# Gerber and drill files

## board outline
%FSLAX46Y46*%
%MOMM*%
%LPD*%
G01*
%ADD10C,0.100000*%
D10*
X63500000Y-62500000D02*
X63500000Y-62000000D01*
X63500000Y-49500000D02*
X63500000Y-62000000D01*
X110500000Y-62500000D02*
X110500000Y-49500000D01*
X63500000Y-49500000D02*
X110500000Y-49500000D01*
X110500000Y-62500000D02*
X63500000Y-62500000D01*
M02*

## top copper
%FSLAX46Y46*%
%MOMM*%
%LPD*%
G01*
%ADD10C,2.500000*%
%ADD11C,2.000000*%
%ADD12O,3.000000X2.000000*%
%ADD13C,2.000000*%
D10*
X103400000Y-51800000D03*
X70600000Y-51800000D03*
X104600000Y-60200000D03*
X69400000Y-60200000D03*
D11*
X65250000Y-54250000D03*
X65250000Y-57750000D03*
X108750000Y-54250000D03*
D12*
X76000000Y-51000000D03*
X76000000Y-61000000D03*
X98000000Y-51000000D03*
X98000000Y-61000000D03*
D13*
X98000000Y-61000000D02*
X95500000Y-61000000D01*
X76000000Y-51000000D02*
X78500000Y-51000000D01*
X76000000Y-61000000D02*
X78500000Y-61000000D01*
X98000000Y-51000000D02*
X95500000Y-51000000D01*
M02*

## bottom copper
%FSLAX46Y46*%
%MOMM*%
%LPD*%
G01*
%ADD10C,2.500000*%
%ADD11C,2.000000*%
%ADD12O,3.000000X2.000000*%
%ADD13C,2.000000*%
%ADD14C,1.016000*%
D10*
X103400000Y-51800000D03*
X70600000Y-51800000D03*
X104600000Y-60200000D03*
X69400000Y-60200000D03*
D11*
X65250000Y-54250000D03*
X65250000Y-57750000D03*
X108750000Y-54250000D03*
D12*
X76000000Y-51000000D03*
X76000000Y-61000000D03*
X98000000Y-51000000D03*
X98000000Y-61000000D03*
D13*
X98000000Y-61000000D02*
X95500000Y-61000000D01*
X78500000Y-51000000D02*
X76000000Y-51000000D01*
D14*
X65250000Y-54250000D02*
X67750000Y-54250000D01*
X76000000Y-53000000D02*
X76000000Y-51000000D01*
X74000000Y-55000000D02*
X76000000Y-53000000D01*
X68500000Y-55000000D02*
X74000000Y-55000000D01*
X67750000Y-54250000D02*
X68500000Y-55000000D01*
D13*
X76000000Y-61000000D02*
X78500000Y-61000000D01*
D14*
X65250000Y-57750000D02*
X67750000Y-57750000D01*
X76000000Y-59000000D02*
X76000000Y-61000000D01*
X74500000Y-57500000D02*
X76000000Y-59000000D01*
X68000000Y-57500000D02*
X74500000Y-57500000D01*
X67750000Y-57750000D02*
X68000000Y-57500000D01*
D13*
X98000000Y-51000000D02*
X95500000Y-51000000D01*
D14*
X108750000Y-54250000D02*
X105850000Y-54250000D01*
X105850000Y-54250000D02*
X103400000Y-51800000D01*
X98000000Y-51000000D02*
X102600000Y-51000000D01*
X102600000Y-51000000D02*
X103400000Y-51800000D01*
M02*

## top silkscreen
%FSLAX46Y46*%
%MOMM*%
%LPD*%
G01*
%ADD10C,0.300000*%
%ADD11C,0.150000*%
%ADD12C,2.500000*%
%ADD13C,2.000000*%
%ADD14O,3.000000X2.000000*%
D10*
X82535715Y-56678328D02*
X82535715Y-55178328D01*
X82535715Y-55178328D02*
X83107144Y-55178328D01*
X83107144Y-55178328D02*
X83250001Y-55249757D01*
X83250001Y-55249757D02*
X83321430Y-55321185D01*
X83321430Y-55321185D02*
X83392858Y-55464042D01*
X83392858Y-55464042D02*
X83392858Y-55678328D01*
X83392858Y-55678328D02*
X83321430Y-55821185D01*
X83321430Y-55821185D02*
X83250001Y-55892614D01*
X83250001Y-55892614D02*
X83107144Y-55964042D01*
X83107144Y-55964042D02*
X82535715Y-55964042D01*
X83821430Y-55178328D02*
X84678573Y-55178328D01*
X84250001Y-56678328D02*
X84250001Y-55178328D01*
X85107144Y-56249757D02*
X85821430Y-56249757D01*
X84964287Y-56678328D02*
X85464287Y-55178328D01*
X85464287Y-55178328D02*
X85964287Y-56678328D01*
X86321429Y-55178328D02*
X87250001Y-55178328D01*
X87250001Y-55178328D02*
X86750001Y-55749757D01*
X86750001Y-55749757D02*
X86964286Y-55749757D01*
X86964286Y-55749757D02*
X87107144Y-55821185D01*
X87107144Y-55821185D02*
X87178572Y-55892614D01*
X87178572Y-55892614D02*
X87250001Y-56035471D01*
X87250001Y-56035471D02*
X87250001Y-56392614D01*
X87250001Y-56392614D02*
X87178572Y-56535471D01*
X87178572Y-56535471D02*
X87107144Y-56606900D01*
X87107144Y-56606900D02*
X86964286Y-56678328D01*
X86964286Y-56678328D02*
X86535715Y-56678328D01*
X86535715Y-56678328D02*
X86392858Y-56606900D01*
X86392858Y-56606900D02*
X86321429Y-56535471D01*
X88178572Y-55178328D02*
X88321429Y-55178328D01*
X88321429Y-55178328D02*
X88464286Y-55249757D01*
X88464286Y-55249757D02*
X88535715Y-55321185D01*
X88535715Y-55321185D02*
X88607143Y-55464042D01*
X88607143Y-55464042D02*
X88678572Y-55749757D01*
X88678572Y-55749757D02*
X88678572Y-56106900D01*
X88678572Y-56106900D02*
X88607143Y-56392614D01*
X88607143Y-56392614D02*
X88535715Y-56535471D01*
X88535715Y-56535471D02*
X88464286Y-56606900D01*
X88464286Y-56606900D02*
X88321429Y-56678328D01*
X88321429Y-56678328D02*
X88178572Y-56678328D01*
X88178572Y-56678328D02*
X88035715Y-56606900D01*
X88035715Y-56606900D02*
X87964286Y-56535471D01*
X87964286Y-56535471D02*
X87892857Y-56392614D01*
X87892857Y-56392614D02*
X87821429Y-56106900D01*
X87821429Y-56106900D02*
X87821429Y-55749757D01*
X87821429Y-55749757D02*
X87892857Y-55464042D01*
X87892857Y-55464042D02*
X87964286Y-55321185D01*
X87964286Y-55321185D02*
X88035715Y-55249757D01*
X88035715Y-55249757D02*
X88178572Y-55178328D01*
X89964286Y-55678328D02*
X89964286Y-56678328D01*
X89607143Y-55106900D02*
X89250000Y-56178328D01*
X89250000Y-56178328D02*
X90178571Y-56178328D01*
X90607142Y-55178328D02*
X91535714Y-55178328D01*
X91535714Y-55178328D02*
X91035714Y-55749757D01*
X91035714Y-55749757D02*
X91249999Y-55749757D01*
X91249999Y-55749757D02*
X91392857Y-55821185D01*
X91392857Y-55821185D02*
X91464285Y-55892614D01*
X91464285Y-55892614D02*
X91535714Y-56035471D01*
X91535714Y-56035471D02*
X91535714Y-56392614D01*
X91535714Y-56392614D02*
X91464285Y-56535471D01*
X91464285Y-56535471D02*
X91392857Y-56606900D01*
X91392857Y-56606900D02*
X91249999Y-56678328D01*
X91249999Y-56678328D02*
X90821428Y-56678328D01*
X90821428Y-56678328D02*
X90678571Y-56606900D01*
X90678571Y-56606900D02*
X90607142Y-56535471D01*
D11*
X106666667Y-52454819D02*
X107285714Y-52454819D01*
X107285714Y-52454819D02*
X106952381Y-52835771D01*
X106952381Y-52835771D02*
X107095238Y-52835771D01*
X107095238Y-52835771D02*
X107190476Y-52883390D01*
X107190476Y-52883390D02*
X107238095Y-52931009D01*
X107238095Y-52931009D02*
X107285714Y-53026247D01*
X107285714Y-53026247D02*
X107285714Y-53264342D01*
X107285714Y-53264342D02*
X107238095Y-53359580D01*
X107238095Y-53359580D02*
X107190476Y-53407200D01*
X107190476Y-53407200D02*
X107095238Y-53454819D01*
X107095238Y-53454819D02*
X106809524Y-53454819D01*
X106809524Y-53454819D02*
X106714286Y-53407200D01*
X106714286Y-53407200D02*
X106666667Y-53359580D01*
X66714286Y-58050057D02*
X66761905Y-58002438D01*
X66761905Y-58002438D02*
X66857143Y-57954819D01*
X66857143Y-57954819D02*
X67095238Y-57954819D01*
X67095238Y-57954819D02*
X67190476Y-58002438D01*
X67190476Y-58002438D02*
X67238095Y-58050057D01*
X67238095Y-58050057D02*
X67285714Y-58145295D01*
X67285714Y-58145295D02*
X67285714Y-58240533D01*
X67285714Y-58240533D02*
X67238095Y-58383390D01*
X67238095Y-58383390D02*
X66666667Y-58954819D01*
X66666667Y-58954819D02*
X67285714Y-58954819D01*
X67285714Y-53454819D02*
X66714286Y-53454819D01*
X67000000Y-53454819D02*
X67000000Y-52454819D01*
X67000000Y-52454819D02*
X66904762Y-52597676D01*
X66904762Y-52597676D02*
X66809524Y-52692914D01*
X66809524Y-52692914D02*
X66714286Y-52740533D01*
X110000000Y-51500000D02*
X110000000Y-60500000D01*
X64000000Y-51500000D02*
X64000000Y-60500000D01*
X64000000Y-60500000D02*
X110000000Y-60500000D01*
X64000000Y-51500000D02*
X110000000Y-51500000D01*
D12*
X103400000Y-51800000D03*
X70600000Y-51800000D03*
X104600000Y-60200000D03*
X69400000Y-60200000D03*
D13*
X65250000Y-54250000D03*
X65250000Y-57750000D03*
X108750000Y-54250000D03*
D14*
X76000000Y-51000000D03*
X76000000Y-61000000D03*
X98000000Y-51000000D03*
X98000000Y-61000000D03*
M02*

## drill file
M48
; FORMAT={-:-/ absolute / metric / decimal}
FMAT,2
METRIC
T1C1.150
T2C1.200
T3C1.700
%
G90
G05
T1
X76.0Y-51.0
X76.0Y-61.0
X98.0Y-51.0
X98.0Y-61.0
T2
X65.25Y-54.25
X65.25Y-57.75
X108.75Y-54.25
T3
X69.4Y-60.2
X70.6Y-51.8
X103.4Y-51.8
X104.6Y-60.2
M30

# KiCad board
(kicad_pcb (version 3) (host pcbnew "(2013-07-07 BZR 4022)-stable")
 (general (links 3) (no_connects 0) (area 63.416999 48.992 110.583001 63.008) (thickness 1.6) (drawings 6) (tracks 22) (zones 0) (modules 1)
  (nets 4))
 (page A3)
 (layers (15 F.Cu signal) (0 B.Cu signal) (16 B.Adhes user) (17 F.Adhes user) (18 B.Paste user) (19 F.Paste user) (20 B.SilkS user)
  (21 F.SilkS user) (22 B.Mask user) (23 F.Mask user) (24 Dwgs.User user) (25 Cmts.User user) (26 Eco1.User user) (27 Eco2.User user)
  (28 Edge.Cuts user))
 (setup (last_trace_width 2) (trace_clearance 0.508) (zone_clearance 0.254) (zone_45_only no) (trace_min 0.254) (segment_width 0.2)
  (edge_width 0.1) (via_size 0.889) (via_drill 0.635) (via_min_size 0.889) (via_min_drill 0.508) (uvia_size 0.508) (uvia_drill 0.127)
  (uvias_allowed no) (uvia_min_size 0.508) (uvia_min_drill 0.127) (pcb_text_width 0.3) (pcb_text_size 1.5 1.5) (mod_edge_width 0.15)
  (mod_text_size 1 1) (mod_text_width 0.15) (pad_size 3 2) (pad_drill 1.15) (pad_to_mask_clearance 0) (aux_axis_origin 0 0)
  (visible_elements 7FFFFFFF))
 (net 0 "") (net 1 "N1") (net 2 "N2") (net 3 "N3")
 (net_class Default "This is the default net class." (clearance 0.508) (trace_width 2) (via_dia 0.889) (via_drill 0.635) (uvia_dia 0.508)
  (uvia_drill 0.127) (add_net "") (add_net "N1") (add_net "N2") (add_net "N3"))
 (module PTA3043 (layer F.Cu) (at 87 56)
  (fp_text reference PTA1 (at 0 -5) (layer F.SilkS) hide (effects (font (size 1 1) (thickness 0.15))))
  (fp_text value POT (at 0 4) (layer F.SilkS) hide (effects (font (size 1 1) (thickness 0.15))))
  (fp_line (start 23 -4.5) (end 23 4.5) (layer F.SilkS) (width 0.15))
  (fp_line (start -23 -4.5) (end -23 4.5) (layer F.SilkS) (width 0.15))
  (fp_line (start -23 4.5) (end 23 4.5) (layer F.SilkS) (width 0.15))
  (fp_line (start -23 -4.5) (end 23 -4.5) (layer F.SilkS) (width 0.15))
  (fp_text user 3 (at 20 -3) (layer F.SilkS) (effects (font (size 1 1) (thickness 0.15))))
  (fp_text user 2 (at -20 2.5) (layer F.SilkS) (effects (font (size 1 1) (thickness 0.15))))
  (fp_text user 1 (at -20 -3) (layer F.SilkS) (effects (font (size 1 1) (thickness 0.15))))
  (pad 7 thru_hole circle (at 16.4 -4.2) (size 2.5 2.5) (drill 1.7) (layers *.Cu *.Mask F.SilkS))
  (pad 6 thru_hole circle (at -16.4 -4.2) (size 2.5 2.5) (drill 1.7) (layers *.Cu *.Mask F.SilkS))
  (pad 5 thru_hole circle (at 17.6 4.2) (size 2.5 2.5) (drill 1.7) (layers *.Cu *.Mask F.SilkS))
  (pad 4 thru_hole circle (at -17.6 4.2) (size 2.5 2.5) (drill 1.7) (layers *.Cu *.Mask F.SilkS))
  (pad 1 thru_hole circle (at -21.75 -1.75) (size 2 2) (drill 1.2) (layers *.Cu *.Mask F.SilkS) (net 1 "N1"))
  (pad 2 thru_hole circle (at -21.75 1.75) (size 2 2) (drill 1.2) (layers *.Cu *.Mask F.SilkS) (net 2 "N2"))
  (pad 3 thru_hole circle (at 21.75 -1.75) (size 2 2) (drill 1.2) (layers *.Cu *.Mask F.SilkS) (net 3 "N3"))
  (pad 1 thru_hole oval (at -11 -5) (size 3 2) (drill 1.15) (layers *.Cu *.Mask F.SilkS) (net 1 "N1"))
  (pad 2 thru_hole oval (at -11 5) (size 3 2) (drill 1.15) (layers *.Cu *.Mask F.SilkS) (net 2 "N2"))
  (pad 3 thru_hole oval (at 11 -5) (size 3 2) (drill 1.15) (layers *.Cu *.Mask F.SilkS) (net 3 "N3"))
  (pad 8 thru_hole oval (at 11 5) (size 3 2) (drill 1.15) (layers *.Cu *.Mask F.SilkS)))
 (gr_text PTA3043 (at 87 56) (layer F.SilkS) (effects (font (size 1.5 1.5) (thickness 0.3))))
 (gr_line (start 63.5 62.5) (end 63.5 62) (angle 90) (layer Edge.Cuts) (width 0.1))
 (gr_line (start 63.5 49.5) (end 63.5 62) (angle 90) (layer Edge.Cuts) (width 0.1))
 (gr_line (start 110.5 62.5) (end 110.5 49.5) (angle 90) (layer Edge.Cuts) (width 0.1))
 (gr_line (start 63.5 49.5) (end 110.5 49.5) (angle 90) (layer Edge.Cuts) (width 0.1))
 (gr_line (start 110.5 62.5) (end 63.5 62.5) (angle 90) (layer Edge.Cuts) (width 0.1))
 (segment (start 98 61) (end 95.5 61) (width 2) (layer F.Cu) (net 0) (status 400000))
 (segment (start 98 61) (end 95.5 61) (width 2) (layer B.Cu) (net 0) (status 400000))
 (segment (start 76 51) (end 78.5 51) (width 2) (layer F.Cu) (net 1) (status 400000))
 (segment (start 78.5 51) (end 76 51) (width 2) (layer B.Cu) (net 1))
 (segment (start 65.25 54.25) (end 67.75 54.25) (width 1.016) (layer B.Cu) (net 1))
 (segment (start 76 53) (end 76 51) (width 1.016) (layer B.Cu) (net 1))
 (segment (start 74 55) (end 76 53) (width 1.016) (layer B.Cu) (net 1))
 (segment (start 68.5 55) (end 74 55) (width 1.016) (layer B.Cu) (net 1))
 (segment (start 67.75 54.25) (end 68.5 55) (width 1.016) (layer B.Cu) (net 1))
 (segment (start 76 61) (end 78.5 61) (width 2) (layer F.Cu) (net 2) (status 400000))
 (segment (start 76 61) (end 78.5 61) (width 2) (layer B.Cu) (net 2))
 (segment (start 65.25 57.75) (end 67.75 57.75) (width 1.016) (layer B.Cu) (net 2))
 (segment (start 76 59) (end 76 61) (width 1.016) (layer B.Cu) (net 2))
 (segment (start 74.5 57.5) (end 76 59) (width 1.016) (layer B.Cu) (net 2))
 (segment (start 68 57.5) (end 74.5 57.5) (width 1.016) (layer B.Cu) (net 2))
 (segment (start 67.75 57.75) (end 68 57.5) (width 1.016) (layer B.Cu) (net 2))
 (segment (start 98 51) (end 95.5 51) (width 2) (layer F.Cu) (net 3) (status 400000))
 (segment (start 98 51) (end 95.5 51) (width 2) (layer B.Cu) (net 3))
 (segment (start 108.75 54.25) (end 105.85 54.25) (width 1.016) (layer B.Cu) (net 3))
 (segment (start 105.85 54.25) (end 103.4 51.8) (width 1.016) (layer B.Cu) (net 3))
 (segment (start 98 51) (end 102.6 51) (width 1.016) (layer B.Cu) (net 3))
 (segment (start 102.6 51) (end 103.4 51.8) (width 1.016) (layer B.Cu) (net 3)))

